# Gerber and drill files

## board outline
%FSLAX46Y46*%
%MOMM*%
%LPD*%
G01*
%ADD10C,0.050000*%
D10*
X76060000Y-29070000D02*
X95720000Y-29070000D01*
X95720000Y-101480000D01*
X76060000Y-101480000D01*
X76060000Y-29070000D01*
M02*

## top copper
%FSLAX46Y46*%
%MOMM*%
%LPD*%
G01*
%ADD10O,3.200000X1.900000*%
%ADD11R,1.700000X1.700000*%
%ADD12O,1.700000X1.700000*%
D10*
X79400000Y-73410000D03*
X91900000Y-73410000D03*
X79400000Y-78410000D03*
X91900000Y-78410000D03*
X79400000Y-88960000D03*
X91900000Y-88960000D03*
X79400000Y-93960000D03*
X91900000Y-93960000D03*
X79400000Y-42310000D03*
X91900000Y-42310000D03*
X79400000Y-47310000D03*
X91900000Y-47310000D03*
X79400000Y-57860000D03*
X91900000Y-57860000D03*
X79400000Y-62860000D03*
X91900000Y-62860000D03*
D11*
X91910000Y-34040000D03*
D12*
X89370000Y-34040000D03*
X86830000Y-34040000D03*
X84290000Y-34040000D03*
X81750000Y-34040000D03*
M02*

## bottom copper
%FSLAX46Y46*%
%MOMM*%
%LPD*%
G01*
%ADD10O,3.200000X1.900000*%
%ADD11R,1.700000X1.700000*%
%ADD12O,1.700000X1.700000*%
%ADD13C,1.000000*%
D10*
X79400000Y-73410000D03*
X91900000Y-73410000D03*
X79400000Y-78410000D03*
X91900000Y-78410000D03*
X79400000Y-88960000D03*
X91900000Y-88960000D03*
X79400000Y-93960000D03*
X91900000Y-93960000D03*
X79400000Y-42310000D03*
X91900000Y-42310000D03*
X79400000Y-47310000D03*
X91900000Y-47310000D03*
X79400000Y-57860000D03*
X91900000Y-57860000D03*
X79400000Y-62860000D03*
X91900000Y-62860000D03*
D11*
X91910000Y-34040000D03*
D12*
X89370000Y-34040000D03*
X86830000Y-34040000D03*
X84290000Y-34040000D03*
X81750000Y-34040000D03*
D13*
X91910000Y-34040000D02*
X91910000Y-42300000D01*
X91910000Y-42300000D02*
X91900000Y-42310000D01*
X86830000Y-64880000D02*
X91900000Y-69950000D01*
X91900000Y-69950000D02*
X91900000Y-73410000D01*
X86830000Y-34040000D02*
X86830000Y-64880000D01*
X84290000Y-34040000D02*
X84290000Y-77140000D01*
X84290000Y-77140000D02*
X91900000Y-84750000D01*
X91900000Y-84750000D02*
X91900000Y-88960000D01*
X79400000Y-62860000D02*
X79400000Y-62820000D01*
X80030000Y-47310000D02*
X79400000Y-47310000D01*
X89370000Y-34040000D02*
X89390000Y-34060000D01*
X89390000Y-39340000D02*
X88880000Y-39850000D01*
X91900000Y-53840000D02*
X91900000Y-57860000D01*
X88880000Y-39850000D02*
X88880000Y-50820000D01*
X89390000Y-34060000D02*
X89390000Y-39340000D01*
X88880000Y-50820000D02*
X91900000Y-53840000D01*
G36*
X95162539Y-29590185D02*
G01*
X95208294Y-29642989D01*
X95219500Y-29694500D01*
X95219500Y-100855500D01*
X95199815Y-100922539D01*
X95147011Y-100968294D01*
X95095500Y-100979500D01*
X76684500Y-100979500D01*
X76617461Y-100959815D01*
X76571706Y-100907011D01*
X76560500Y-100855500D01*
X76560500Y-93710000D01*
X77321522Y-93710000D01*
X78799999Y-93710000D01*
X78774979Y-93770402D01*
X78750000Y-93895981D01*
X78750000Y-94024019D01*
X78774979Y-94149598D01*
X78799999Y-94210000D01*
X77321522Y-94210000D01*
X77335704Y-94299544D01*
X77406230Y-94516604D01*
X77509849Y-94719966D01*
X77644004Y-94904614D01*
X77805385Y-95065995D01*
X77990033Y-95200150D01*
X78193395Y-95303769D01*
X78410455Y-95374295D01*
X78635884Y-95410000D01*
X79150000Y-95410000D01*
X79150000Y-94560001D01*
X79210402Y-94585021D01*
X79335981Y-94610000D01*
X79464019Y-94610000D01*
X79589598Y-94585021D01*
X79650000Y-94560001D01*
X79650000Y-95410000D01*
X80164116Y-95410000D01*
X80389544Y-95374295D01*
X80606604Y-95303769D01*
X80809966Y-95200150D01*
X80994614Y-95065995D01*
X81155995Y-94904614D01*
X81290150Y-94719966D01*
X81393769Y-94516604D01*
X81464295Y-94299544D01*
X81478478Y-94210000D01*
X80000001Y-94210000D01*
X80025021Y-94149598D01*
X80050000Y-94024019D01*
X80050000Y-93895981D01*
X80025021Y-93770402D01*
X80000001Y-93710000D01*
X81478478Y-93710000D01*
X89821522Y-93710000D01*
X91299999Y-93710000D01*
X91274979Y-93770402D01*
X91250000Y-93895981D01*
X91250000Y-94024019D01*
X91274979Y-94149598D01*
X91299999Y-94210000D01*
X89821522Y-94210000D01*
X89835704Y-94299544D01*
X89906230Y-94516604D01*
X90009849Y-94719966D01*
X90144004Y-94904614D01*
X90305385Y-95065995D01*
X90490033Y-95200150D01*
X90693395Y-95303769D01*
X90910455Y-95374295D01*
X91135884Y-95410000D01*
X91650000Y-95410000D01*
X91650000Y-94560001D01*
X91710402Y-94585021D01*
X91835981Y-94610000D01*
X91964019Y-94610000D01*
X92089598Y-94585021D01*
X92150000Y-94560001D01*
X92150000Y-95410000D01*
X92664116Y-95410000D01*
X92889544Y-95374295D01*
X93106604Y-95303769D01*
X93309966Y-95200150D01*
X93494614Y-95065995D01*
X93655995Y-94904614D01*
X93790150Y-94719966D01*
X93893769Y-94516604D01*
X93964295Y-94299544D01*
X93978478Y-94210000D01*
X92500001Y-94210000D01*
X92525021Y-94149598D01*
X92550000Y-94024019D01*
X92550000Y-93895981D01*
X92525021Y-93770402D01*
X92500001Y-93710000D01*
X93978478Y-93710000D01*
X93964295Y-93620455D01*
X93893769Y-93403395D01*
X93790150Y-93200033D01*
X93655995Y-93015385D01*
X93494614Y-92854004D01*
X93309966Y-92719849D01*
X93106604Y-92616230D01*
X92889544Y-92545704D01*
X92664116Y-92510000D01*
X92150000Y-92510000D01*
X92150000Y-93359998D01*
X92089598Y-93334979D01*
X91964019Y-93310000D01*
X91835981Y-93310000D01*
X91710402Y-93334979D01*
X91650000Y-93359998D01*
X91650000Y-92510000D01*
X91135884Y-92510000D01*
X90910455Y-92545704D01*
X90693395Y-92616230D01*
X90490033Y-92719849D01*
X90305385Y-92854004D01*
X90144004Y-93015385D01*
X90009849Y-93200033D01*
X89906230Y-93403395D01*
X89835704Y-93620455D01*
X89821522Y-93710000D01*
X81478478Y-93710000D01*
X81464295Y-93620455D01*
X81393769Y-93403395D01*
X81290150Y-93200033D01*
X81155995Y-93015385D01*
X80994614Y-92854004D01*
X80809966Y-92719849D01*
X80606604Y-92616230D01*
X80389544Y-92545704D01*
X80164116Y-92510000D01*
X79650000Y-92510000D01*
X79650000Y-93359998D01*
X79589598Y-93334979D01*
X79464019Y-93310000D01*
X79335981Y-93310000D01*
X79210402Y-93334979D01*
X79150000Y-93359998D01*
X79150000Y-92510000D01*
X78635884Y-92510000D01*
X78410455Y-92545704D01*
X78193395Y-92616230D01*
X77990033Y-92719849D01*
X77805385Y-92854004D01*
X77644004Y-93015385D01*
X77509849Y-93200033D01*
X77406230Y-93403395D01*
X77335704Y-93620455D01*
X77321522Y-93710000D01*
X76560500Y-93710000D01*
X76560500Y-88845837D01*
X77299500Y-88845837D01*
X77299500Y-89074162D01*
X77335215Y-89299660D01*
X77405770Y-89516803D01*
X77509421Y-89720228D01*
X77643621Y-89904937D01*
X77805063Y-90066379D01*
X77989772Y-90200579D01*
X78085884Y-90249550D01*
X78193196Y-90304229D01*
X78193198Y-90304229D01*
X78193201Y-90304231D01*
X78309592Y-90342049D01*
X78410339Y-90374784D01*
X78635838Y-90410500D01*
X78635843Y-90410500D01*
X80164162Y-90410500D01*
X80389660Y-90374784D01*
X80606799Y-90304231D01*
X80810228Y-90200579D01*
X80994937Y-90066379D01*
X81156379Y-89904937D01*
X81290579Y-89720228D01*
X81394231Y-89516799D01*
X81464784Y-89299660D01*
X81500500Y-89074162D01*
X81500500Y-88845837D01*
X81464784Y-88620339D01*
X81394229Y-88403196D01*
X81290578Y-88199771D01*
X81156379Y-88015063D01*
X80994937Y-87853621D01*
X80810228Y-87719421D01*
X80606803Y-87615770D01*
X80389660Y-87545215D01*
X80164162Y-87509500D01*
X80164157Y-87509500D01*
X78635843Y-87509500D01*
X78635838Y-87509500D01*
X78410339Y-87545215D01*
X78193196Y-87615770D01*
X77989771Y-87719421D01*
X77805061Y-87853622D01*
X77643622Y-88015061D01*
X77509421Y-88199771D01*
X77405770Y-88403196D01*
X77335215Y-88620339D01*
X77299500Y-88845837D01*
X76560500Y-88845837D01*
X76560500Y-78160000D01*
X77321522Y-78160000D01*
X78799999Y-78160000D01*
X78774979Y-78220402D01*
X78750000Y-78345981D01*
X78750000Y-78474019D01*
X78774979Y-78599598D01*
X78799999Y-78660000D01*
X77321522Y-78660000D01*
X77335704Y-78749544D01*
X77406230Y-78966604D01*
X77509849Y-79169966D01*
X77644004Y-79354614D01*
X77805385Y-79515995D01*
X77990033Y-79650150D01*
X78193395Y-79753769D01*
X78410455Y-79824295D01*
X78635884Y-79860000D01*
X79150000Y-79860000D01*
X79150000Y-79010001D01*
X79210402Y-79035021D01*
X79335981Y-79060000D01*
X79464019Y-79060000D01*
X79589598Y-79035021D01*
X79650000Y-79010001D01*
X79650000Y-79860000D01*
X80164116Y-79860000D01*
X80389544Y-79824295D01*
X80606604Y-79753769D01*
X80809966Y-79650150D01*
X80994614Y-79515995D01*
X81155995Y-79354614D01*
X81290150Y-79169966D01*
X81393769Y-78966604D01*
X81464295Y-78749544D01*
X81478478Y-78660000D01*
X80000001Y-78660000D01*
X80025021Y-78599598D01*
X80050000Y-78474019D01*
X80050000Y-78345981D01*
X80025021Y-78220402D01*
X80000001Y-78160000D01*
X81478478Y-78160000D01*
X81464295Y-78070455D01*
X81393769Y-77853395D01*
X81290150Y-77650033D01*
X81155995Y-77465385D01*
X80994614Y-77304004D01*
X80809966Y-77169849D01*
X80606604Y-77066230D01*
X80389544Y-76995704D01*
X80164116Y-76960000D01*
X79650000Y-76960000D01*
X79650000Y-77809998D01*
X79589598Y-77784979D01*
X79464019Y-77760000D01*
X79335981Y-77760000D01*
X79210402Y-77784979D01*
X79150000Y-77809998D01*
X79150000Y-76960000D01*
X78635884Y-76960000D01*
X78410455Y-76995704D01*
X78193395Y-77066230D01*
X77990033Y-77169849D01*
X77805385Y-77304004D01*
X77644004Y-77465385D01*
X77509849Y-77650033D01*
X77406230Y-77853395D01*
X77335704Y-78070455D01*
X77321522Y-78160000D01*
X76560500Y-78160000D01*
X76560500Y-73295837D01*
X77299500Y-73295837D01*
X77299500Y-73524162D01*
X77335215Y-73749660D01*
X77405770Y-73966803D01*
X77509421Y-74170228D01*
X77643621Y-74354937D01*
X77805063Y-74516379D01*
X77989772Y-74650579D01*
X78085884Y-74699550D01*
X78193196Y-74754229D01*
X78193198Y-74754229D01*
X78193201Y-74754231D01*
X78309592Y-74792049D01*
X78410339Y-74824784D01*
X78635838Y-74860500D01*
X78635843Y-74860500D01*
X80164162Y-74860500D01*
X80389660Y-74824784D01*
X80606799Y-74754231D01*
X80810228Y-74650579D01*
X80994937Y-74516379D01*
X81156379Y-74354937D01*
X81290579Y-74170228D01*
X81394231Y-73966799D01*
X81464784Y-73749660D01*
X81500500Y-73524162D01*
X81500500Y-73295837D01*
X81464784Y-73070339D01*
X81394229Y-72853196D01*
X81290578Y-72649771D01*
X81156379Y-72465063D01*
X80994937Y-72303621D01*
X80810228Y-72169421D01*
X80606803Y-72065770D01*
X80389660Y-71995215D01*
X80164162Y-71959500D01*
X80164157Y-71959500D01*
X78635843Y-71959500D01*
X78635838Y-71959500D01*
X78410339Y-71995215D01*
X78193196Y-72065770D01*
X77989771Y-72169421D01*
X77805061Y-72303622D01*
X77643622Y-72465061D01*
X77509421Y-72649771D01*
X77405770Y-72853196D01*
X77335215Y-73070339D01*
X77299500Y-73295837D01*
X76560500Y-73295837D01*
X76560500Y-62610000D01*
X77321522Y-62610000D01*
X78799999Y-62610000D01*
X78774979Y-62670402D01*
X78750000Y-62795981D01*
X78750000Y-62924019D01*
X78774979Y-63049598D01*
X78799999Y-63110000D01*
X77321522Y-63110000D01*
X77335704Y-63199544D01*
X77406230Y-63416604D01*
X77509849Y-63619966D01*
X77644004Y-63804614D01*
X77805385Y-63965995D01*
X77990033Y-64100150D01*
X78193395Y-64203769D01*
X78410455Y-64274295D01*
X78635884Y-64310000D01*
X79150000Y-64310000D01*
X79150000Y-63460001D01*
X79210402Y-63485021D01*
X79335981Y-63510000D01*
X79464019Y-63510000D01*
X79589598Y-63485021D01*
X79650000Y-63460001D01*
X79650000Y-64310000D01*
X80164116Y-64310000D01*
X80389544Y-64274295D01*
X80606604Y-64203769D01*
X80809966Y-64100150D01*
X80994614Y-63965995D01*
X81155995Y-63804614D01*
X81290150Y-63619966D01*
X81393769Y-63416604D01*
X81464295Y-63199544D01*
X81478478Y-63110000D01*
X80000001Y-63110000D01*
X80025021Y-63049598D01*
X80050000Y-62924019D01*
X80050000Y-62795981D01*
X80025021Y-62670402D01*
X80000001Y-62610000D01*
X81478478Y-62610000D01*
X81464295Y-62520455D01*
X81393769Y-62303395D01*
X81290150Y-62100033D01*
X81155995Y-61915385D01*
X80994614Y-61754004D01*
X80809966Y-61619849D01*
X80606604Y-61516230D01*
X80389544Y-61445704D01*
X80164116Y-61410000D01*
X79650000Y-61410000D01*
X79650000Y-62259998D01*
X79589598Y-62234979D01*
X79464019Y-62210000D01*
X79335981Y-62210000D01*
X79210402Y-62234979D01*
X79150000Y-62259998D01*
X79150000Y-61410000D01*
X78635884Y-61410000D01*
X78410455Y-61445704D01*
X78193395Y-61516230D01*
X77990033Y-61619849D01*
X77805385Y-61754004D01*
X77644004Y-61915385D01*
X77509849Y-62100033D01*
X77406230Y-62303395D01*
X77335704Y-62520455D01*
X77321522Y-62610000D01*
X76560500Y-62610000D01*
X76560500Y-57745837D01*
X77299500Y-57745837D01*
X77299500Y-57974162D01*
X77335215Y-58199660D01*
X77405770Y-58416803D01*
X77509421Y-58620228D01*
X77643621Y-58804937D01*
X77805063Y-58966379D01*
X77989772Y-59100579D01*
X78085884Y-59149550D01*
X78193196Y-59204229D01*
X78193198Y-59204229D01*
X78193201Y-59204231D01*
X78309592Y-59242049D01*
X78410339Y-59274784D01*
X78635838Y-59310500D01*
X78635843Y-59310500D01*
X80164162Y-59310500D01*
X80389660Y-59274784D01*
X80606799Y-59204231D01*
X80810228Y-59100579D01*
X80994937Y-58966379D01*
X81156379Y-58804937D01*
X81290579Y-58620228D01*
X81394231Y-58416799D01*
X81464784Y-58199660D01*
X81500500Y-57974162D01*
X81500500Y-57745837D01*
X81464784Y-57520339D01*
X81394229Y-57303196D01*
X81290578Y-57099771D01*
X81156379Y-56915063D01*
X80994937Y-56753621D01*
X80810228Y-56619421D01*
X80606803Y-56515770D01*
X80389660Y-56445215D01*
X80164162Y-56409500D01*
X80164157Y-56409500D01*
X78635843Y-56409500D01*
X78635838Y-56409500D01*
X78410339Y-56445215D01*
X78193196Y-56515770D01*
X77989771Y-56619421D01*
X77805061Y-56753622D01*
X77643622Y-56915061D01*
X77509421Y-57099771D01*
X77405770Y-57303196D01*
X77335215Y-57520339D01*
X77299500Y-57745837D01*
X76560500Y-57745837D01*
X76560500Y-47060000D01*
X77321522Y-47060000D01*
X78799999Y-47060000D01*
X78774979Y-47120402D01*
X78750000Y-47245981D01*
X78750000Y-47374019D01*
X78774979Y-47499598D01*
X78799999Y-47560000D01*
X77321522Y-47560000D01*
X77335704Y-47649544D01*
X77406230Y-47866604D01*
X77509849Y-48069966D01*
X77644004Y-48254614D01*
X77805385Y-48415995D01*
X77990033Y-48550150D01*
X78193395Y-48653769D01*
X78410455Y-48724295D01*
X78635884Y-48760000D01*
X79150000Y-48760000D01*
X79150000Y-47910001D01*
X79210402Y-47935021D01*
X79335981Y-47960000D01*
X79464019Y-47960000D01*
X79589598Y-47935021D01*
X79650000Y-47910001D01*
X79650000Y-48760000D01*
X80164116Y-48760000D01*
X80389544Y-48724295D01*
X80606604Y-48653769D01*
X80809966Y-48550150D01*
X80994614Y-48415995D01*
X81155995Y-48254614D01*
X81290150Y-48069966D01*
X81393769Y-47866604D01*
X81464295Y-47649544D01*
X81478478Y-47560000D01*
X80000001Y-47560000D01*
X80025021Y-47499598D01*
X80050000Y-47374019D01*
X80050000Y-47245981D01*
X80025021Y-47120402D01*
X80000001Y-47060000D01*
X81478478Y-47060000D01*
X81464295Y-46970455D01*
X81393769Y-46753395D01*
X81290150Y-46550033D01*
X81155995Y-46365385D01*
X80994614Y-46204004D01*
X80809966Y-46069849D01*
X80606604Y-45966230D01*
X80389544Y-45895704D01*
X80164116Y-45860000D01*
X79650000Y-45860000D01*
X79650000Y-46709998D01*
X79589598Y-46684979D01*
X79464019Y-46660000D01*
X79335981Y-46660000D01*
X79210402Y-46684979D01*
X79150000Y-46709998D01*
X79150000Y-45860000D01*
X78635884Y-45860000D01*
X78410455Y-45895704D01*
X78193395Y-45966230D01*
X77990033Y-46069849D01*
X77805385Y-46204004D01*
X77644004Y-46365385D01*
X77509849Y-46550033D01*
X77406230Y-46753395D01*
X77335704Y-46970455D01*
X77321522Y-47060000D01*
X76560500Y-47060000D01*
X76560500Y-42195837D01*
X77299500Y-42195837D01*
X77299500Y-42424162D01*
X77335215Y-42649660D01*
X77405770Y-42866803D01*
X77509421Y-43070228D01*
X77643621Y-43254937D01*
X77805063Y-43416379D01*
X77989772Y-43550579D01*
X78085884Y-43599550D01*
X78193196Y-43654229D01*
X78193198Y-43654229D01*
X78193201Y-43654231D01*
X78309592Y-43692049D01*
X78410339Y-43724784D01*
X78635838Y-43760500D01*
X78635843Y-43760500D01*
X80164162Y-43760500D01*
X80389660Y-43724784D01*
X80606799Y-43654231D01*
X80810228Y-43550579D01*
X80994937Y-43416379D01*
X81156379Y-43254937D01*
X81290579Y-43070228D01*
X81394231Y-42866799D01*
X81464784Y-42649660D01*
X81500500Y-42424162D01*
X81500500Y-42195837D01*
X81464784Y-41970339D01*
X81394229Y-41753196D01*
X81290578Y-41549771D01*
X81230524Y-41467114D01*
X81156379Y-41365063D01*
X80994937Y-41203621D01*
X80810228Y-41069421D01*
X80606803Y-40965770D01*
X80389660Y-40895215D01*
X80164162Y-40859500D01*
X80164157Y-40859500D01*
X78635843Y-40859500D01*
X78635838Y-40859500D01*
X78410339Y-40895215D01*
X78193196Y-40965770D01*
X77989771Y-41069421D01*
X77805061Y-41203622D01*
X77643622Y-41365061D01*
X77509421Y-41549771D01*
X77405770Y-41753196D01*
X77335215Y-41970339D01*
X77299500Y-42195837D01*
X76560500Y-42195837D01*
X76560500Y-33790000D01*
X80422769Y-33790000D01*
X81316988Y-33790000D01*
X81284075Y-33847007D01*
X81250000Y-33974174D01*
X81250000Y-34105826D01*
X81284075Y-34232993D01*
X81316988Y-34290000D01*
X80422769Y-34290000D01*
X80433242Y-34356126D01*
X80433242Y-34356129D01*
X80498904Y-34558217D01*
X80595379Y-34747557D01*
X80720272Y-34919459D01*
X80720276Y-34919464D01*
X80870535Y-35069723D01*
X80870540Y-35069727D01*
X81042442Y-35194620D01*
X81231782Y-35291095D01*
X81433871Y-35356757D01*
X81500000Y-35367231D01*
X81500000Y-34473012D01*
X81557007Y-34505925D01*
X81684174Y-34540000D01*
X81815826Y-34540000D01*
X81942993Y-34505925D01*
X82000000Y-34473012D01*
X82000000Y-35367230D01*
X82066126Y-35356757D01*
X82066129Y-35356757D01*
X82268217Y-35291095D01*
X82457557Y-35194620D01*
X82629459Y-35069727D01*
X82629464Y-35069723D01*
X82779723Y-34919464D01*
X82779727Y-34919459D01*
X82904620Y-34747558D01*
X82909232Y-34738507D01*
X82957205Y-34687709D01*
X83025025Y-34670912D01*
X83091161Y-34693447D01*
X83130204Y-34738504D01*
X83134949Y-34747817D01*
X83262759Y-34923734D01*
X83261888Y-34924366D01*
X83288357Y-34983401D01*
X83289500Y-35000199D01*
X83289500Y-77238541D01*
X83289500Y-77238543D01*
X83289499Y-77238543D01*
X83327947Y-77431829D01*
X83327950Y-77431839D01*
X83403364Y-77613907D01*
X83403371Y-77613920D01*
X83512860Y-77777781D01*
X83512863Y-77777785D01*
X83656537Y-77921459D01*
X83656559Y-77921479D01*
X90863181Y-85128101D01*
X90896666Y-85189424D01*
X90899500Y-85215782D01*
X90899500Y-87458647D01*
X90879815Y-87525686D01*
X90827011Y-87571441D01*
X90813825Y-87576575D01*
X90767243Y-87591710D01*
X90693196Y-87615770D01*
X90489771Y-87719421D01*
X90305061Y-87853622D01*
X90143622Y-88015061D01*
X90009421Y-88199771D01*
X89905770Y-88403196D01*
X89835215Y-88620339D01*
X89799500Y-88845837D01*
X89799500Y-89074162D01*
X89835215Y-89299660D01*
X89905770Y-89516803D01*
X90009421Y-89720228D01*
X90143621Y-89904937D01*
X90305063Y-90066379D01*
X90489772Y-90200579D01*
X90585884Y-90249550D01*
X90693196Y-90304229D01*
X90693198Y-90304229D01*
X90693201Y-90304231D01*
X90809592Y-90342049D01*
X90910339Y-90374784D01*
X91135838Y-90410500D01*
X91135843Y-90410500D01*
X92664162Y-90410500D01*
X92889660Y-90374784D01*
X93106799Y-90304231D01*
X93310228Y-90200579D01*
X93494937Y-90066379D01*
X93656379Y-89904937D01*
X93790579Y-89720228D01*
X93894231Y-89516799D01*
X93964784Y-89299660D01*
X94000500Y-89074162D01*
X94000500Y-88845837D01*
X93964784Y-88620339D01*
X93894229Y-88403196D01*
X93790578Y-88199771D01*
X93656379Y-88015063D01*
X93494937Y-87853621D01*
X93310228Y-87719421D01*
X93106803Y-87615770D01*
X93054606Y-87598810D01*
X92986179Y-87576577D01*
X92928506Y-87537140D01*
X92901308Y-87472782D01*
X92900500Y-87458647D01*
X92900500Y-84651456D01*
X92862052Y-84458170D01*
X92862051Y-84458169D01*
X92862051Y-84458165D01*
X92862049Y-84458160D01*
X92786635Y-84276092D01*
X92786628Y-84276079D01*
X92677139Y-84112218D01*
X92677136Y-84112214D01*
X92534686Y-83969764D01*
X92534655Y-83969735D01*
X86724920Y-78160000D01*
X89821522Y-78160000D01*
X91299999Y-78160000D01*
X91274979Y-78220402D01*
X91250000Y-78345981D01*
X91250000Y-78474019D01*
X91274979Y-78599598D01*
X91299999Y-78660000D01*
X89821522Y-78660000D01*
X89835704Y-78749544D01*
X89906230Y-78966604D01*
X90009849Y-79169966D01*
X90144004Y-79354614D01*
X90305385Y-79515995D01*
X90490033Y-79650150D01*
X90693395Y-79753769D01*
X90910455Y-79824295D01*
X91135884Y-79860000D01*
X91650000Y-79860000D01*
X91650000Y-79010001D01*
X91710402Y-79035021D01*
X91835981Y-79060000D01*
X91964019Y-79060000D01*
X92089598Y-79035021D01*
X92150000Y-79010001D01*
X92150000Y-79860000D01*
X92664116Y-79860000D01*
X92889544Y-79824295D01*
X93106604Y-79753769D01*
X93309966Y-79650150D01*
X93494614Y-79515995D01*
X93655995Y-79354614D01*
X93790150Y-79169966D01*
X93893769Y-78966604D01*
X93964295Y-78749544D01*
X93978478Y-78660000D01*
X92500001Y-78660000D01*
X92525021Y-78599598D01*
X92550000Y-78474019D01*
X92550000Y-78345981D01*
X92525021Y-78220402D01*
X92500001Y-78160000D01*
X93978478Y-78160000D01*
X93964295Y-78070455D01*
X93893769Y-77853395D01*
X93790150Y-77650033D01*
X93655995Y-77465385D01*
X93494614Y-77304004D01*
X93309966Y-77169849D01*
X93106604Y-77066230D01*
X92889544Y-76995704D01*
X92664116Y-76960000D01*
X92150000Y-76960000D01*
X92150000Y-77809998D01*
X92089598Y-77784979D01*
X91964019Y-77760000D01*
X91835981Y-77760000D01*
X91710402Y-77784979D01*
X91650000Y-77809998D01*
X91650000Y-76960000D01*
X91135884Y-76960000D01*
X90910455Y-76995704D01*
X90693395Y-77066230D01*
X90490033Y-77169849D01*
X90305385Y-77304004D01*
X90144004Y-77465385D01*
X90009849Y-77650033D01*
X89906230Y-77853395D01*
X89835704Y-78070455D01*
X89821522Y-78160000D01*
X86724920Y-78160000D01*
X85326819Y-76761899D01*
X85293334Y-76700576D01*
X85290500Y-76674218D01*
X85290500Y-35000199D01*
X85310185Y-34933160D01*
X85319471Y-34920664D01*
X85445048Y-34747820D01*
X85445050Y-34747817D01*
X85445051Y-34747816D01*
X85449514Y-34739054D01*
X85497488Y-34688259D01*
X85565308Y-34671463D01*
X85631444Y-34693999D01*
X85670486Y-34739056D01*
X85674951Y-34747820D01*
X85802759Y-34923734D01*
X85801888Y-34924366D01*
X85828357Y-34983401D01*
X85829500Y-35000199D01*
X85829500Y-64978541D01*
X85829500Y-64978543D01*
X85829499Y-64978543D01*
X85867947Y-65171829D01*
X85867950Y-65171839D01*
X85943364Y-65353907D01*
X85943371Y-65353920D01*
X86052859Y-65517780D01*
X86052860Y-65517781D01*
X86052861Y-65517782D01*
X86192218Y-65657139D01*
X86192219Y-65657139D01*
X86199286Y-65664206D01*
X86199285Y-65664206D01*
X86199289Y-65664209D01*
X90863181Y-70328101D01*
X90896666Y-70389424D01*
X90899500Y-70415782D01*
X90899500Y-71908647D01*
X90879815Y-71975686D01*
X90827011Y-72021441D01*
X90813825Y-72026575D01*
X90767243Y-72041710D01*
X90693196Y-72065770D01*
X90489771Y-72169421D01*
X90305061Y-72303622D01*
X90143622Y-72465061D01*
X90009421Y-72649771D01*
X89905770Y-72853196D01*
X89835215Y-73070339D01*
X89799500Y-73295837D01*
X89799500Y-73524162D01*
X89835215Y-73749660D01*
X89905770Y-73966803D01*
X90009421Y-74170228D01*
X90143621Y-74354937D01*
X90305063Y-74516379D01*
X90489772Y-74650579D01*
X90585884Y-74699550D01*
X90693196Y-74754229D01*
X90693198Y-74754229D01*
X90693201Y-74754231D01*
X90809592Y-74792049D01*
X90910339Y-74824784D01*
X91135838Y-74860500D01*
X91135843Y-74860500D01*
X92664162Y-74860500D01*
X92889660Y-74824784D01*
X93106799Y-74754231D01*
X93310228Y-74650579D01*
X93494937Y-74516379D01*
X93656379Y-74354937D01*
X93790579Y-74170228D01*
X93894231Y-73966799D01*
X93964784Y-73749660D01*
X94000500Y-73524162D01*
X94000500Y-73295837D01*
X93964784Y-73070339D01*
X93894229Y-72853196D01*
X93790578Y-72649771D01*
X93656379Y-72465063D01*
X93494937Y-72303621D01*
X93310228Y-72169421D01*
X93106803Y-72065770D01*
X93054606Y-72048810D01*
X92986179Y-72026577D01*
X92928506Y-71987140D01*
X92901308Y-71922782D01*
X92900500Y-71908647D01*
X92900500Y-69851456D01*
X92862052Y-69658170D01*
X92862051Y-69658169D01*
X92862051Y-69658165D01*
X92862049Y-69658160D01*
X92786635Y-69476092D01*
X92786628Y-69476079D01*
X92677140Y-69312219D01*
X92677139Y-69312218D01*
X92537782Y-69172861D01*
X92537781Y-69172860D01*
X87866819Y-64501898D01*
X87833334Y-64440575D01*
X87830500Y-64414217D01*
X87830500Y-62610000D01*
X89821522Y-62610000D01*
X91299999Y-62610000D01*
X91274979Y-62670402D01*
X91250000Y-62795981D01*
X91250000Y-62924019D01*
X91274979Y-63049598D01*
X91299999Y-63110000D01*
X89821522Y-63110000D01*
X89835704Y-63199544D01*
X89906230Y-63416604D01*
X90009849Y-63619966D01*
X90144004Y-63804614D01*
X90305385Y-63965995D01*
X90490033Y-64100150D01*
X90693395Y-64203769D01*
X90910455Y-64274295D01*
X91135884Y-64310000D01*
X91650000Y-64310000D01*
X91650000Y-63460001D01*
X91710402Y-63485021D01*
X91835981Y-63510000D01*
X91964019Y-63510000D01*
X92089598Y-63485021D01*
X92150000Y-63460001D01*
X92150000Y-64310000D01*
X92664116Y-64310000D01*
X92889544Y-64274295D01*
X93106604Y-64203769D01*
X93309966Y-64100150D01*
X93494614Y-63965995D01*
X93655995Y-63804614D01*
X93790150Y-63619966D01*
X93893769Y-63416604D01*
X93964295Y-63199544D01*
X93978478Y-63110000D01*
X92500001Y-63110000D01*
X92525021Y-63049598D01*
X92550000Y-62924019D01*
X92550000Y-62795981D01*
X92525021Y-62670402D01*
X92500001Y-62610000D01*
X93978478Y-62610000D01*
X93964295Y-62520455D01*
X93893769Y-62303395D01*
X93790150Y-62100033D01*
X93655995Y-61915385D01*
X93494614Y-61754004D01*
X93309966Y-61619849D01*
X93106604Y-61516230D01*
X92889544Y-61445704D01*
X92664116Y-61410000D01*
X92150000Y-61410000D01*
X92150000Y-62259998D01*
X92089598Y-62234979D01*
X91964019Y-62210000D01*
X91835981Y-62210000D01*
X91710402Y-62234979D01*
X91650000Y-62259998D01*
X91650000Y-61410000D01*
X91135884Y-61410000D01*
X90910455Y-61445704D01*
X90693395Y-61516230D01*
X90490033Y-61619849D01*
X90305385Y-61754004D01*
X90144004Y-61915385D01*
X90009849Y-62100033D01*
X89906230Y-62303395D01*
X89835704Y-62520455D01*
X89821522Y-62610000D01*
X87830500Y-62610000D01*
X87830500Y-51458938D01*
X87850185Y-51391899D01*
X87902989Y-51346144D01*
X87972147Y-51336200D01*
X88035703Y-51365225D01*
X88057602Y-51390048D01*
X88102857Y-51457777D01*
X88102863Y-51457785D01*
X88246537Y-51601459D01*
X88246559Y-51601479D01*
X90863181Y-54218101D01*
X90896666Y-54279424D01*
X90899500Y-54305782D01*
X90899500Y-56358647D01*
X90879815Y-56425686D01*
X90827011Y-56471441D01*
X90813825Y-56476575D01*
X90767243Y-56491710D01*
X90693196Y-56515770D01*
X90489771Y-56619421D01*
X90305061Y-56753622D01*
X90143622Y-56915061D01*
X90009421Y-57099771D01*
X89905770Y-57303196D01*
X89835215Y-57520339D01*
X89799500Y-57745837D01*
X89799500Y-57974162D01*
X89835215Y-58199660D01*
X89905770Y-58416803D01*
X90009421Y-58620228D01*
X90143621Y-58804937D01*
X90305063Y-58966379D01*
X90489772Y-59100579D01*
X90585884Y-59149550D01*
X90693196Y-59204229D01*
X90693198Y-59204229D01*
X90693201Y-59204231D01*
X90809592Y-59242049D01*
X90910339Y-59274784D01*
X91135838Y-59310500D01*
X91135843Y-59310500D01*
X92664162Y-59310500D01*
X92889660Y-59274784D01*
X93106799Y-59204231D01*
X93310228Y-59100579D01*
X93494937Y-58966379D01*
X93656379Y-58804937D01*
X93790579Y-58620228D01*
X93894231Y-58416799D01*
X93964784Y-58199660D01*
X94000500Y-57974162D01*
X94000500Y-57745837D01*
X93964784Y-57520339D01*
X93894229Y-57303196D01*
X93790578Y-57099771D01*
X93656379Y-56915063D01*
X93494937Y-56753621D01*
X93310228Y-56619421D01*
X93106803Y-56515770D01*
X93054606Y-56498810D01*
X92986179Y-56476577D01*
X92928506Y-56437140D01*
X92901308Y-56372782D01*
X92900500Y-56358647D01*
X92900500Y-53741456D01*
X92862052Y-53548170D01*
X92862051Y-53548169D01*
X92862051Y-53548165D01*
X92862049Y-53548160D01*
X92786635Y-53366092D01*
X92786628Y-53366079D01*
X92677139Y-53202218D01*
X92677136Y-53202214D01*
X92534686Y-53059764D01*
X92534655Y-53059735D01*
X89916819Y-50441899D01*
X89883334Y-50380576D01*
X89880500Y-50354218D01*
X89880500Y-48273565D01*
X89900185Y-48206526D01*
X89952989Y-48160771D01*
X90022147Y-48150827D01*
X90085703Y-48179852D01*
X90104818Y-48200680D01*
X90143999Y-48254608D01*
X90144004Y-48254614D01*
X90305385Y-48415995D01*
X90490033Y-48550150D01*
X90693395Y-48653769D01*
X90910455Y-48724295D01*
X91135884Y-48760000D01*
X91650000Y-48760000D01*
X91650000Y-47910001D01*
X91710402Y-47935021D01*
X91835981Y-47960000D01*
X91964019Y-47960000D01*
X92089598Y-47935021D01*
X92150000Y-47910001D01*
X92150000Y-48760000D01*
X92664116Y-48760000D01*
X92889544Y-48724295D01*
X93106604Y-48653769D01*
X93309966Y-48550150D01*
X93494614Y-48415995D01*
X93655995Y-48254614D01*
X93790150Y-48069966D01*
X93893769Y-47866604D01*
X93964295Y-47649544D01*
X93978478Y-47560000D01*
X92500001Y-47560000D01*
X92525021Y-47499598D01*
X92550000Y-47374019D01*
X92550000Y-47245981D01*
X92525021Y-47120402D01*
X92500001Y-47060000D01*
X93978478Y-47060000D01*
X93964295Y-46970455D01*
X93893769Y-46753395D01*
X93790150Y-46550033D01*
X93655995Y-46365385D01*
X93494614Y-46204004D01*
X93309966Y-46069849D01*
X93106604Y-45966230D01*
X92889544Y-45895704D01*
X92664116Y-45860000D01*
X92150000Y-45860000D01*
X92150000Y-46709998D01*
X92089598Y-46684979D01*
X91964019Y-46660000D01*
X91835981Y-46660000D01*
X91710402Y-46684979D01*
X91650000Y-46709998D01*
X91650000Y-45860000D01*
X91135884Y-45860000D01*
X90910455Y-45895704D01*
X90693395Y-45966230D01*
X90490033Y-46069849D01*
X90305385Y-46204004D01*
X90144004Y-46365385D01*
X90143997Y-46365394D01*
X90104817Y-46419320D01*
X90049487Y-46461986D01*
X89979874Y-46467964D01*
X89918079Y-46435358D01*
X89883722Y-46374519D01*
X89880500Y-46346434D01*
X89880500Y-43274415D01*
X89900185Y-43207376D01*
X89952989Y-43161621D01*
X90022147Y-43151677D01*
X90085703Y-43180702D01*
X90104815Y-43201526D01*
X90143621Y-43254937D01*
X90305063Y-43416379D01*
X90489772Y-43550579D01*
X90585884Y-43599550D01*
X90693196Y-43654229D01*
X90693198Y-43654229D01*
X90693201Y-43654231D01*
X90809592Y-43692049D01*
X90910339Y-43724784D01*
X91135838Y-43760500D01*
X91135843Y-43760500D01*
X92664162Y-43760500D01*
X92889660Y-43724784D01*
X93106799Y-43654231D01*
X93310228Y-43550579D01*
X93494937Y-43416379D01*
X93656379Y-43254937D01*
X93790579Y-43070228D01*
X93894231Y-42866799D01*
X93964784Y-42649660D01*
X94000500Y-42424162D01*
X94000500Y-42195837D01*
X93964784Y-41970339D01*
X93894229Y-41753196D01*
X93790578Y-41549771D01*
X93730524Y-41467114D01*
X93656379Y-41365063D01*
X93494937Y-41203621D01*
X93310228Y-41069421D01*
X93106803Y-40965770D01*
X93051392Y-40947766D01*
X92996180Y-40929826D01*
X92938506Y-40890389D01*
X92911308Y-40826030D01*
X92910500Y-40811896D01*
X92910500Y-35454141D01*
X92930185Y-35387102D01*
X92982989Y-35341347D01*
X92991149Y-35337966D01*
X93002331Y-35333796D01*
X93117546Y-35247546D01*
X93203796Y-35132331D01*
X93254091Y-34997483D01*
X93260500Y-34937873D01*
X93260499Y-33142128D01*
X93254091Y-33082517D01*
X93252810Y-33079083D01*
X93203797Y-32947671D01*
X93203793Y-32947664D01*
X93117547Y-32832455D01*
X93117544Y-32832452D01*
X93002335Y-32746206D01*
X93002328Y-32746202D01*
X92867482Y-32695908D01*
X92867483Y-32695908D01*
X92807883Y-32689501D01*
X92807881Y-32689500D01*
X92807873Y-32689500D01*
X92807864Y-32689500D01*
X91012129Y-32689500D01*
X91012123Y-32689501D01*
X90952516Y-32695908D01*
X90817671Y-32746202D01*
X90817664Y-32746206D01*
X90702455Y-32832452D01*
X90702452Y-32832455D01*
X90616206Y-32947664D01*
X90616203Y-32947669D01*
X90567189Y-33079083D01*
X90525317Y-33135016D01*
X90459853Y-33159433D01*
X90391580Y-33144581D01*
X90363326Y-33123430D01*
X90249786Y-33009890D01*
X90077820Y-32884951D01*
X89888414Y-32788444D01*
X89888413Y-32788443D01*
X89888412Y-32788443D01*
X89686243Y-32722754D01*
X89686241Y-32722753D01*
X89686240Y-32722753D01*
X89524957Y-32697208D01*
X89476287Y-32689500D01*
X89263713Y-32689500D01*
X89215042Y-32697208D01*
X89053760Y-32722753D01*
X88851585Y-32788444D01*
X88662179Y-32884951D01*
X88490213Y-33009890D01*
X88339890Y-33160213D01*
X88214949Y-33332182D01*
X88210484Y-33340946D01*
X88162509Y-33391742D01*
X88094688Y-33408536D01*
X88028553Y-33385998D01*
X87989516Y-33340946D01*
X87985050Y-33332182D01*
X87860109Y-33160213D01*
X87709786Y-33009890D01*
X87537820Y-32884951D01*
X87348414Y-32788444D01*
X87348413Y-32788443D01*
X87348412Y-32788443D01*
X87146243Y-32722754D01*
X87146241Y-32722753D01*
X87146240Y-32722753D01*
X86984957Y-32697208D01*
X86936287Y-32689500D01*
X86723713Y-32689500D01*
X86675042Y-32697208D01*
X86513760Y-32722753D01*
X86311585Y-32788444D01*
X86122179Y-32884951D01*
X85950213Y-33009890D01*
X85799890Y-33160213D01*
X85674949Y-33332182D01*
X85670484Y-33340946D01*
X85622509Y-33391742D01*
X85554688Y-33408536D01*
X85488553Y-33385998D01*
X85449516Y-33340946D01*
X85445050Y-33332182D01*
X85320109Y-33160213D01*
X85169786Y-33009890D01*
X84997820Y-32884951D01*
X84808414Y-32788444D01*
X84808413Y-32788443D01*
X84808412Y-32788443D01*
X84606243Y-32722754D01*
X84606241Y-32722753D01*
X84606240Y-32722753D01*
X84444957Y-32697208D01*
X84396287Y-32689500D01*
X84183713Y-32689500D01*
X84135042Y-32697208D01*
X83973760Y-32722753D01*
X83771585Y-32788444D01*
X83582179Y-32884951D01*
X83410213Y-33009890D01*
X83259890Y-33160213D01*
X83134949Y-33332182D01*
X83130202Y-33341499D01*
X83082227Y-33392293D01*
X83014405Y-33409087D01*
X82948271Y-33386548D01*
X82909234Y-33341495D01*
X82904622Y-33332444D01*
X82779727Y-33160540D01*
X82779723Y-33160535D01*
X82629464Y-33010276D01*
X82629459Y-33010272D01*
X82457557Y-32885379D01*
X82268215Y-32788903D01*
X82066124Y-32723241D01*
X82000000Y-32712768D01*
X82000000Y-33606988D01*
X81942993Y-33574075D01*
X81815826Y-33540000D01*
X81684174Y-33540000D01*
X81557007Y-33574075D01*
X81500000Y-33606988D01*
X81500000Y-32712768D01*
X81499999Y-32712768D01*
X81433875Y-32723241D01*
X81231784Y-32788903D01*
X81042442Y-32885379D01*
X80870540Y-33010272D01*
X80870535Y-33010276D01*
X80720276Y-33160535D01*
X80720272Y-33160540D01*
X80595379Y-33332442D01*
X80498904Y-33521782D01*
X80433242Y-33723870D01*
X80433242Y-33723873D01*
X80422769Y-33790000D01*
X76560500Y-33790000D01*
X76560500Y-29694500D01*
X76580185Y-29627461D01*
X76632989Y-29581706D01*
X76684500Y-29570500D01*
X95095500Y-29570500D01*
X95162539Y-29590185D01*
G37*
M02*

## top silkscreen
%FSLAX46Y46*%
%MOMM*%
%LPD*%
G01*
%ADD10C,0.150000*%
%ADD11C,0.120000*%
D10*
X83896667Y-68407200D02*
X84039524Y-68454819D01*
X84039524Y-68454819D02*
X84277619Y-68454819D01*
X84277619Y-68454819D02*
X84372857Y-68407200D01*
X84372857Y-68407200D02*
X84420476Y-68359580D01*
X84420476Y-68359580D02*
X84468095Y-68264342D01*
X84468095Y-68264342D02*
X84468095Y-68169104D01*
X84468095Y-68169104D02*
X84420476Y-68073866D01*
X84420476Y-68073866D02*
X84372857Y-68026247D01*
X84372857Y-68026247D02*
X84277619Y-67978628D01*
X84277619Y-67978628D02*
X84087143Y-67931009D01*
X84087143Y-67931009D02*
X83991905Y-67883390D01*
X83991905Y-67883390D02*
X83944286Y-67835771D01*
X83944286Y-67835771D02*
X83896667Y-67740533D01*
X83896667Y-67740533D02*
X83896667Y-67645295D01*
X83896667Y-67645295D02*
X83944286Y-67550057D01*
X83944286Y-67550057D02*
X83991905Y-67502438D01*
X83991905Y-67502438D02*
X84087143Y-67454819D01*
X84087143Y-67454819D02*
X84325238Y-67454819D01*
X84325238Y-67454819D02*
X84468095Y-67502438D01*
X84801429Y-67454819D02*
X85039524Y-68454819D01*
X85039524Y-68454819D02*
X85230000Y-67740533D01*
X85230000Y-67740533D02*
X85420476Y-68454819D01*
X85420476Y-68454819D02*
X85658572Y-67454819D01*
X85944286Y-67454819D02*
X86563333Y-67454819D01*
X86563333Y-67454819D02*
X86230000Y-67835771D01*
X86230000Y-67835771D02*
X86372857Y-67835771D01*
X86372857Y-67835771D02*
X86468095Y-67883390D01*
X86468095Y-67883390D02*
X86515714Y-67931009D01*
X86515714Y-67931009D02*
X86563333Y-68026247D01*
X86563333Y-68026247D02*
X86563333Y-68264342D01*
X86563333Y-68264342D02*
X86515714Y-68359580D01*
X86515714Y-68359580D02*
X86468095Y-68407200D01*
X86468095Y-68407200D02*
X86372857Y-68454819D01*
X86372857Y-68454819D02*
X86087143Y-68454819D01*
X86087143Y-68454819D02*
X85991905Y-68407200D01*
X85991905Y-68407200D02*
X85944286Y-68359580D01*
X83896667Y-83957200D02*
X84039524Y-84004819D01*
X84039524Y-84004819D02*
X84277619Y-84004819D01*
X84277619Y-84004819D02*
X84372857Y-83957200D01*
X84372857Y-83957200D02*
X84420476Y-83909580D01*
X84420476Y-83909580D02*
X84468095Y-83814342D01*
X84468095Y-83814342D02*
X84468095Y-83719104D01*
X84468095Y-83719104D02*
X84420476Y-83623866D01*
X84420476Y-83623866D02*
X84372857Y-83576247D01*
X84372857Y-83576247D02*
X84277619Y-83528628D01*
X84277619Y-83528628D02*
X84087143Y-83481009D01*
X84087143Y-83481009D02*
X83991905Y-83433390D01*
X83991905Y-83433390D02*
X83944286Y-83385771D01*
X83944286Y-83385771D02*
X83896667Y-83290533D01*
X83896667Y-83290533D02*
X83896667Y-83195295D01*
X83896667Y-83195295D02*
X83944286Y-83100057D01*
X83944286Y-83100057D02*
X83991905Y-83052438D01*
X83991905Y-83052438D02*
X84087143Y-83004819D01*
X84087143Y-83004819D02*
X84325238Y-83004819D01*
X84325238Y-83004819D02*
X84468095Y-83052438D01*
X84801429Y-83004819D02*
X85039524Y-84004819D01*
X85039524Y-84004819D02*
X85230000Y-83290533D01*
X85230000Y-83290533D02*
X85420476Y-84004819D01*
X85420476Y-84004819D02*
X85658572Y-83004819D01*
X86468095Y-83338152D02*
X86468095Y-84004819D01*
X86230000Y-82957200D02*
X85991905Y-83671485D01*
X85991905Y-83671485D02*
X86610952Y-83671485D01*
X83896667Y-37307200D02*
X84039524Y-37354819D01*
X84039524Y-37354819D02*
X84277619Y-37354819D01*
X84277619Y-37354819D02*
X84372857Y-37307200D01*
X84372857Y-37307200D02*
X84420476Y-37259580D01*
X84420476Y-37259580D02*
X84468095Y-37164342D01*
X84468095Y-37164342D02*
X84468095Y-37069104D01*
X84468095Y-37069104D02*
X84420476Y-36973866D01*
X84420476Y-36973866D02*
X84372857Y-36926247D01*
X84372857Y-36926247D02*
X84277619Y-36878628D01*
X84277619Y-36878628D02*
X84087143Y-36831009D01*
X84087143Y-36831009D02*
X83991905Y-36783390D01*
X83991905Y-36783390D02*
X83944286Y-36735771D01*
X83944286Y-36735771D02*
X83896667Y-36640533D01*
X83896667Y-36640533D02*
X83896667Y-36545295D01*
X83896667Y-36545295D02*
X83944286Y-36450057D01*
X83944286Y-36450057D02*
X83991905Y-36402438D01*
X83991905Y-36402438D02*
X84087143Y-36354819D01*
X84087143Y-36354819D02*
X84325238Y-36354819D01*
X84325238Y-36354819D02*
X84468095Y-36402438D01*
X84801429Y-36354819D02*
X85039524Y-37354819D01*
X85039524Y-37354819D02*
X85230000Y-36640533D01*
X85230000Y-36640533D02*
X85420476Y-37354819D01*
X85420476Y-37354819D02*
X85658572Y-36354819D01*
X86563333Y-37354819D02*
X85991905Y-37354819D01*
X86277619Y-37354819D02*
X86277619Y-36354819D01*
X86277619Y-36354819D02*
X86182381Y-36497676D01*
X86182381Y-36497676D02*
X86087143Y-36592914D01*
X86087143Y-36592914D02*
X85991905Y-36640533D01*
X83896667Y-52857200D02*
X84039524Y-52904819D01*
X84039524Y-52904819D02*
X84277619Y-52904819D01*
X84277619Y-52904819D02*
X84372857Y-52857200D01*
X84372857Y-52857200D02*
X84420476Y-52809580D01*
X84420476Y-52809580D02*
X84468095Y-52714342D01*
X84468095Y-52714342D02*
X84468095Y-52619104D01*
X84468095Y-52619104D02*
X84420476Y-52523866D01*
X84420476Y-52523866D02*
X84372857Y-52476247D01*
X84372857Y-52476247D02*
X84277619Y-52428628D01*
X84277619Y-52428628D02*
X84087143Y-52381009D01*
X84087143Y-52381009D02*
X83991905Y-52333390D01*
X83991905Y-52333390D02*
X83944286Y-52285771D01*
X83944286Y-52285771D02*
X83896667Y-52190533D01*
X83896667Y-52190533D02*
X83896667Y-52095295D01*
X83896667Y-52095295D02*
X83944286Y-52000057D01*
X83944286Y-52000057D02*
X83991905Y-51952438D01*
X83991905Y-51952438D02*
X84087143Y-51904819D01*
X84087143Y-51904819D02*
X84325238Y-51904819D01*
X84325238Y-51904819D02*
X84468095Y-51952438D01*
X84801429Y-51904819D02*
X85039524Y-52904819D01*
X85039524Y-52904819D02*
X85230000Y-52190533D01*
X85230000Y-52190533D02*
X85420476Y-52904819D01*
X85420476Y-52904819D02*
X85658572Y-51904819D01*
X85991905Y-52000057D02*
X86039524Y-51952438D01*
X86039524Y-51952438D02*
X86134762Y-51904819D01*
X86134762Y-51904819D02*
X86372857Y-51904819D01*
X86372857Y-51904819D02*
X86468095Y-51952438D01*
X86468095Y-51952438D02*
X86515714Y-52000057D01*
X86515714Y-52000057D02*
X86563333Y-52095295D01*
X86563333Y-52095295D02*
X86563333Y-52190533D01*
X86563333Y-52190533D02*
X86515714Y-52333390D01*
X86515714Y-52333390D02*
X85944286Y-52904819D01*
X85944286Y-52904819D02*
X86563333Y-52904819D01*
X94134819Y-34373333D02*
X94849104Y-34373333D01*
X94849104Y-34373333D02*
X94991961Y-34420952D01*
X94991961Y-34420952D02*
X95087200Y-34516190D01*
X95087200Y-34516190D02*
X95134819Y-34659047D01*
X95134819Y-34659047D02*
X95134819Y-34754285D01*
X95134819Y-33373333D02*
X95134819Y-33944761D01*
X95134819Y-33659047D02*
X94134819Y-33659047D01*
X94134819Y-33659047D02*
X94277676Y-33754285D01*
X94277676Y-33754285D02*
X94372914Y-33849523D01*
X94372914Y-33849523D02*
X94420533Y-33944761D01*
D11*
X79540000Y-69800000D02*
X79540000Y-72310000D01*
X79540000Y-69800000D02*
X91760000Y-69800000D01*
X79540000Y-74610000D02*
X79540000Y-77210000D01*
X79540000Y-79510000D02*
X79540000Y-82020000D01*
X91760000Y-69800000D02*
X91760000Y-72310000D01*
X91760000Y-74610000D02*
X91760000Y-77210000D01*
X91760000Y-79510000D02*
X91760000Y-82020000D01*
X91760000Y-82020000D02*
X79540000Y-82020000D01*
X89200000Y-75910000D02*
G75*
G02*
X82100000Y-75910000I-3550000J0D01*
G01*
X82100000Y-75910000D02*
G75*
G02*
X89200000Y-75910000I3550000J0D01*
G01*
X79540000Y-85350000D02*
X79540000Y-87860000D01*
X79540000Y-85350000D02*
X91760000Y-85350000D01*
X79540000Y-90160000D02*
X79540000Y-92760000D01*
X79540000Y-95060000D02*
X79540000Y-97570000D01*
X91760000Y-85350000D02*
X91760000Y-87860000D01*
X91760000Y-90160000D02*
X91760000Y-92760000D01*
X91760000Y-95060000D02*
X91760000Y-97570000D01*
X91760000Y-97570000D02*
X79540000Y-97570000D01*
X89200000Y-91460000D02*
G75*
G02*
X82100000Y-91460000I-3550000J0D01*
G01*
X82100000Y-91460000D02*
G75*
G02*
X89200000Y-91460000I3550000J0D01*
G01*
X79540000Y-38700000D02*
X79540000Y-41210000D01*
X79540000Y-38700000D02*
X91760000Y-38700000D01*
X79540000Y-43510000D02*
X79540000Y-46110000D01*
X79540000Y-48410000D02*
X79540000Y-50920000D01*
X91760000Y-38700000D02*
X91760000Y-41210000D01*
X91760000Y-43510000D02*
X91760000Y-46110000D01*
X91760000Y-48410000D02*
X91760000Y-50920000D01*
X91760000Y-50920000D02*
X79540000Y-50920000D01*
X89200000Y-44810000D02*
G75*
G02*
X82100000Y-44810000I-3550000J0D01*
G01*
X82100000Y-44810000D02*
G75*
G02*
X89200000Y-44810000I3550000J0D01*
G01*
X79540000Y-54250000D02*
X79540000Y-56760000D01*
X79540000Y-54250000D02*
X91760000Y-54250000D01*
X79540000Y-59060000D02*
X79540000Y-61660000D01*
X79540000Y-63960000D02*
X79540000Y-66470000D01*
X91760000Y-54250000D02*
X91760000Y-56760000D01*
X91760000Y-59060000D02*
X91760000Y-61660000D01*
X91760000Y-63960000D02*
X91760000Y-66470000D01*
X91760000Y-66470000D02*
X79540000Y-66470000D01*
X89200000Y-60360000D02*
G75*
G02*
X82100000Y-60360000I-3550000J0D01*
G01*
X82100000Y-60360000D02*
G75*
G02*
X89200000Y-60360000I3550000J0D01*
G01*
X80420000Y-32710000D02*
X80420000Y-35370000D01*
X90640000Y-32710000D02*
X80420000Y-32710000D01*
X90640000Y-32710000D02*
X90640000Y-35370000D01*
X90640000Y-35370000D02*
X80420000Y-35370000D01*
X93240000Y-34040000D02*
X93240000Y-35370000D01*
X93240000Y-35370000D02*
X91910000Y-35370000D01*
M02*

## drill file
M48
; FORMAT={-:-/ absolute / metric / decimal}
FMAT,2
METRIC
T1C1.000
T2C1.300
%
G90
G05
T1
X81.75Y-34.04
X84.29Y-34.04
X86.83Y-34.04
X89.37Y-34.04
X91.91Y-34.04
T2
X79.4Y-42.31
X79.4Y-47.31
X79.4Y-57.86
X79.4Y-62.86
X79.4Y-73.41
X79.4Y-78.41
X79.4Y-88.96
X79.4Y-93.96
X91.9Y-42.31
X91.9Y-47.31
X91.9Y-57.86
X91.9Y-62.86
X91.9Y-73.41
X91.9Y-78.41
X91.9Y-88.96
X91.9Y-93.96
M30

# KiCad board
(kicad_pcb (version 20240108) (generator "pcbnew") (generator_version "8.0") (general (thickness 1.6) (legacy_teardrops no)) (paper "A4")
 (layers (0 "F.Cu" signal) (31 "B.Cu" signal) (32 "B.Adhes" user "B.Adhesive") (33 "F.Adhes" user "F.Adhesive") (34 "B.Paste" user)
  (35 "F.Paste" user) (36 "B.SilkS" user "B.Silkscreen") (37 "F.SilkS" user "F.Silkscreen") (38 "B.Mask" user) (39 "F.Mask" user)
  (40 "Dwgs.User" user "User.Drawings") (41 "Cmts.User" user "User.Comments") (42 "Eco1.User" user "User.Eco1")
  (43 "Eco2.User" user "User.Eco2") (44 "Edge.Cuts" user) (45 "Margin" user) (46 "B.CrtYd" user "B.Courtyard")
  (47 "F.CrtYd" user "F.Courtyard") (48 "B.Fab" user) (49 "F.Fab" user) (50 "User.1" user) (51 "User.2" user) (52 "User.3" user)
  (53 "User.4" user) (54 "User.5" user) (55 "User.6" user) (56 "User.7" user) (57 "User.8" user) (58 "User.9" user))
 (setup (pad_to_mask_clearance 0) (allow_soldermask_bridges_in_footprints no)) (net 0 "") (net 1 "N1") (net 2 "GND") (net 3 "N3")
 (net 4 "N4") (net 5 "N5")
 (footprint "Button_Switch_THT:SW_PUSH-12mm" (layer "F.Cu") (at 79.4 73.41)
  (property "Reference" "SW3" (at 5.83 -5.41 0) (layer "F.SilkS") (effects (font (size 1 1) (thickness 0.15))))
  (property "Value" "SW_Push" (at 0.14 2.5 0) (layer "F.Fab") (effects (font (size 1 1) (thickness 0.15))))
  (fp_line (start 0.14 -3.61) (end 0.14 -1.1) (stroke (width 0.12) (type default)) (layer "F.SilkS"))
  (fp_line (start 0.14 -3.61) (end 12.36 -3.61) (stroke (width 0.12) (type default)) (layer "F.SilkS"))
  (fp_line (start 0.14 1.2) (end 0.14 3.8) (stroke (width 0.12) (type default)) (layer "F.SilkS"))
  (fp_line (start 0.14 6.1) (end 0.14 8.61) (stroke (width 0.12) (type default)) (layer "F.SilkS"))
  (fp_line (start 12.36 -3.61) (end 12.36 -1.1) (stroke (width 0.12) (type default)) (layer "F.SilkS"))
  (fp_line (start 12.36 1.2) (end 12.36 3.8) (stroke (width 0.12) (type default)) (layer "F.SilkS"))
  (fp_line (start 12.36 6.1) (end 12.36 8.61) (stroke (width 0.12) (type default)) (layer "F.SilkS"))
  (fp_line (start 12.36 8.61) (end 0.14 8.61) (stroke (width 0.12) (type default)) (layer "F.SilkS"))
  (fp_circle (center 6.25 2.5) (end 9.8 2.5) (stroke (width 0.12) (type default)) (fill none) (layer "F.SilkS"))
  (pad "1" thru_hole oval (at 0 0) (size 3.2 1.9) (drill 1.3) (layers "*.Cu" "*.Mask") (remove_unused_layers no) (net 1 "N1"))
  (pad "1" thru_hole oval (at 12.5 0) (size 3.2 1.9) (drill 1.3) (layers "*.Cu" "*.Mask") (remove_unused_layers no) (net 1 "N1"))
  (pad "2" thru_hole oval (at 0 5) (size 3.2 1.9) (drill 1.3) (layers "*.Cu" "*.Mask") (remove_unused_layers no) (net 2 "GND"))
  (pad "2" thru_hole oval (at 12.5 5) (size 3.2 1.9) (drill 1.3) (layers "*.Cu" "*.Mask") (remove_unused_layers no) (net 2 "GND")))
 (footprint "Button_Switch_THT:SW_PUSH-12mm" (layer "F.Cu") (at 79.4 88.96)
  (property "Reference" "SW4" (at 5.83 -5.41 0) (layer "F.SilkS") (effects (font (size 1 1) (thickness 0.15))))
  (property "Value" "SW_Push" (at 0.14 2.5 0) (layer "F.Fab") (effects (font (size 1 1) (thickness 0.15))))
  (fp_line (start 0.14 -3.61) (end 0.14 -1.1) (stroke (width 0.12) (type default)) (layer "F.SilkS"))
  (fp_line (start 0.14 -3.61) (end 12.36 -3.61) (stroke (width 0.12) (type default)) (layer "F.SilkS"))
  (fp_line (start 0.14 1.2) (end 0.14 3.8) (stroke (width 0.12) (type default)) (layer "F.SilkS"))
  (fp_line (start 0.14 6.1) (end 0.14 8.61) (stroke (width 0.12) (type default)) (layer "F.SilkS"))
  (fp_line (start 12.36 -3.61) (end 12.36 -1.1) (stroke (width 0.12) (type default)) (layer "F.SilkS"))
  (fp_line (start 12.36 1.2) (end 12.36 3.8) (stroke (width 0.12) (type default)) (layer "F.SilkS"))
  (fp_line (start 12.36 6.1) (end 12.36 8.61) (stroke (width 0.12) (type default)) (layer "F.SilkS"))
  (fp_line (start 12.36 8.61) (end 0.14 8.61) (stroke (width 0.12) (type default)) (layer "F.SilkS"))
  (fp_circle (center 6.25 2.5) (end 9.8 2.5) (stroke (width 0.12) (type default)) (fill none) (layer "F.SilkS"))
  (pad "1" thru_hole oval (at 0 0) (size 3.2 1.9) (drill 1.3) (layers "*.Cu" "*.Mask") (remove_unused_layers no) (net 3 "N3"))
  (pad "1" thru_hole oval (at 12.5 0) (size 3.2 1.9) (drill 1.3) (layers "*.Cu" "*.Mask") (remove_unused_layers no) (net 3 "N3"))
  (pad "2" thru_hole oval (at 0 5) (size 3.2 1.9) (drill 1.3) (layers "*.Cu" "*.Mask") (remove_unused_layers no) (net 2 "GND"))
  (pad "2" thru_hole oval (at 12.5 5) (size 3.2 1.9) (drill 1.3) (layers "*.Cu" "*.Mask") (remove_unused_layers no) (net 2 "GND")))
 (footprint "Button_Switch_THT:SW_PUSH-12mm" (layer "F.Cu") (at 79.4 42.31)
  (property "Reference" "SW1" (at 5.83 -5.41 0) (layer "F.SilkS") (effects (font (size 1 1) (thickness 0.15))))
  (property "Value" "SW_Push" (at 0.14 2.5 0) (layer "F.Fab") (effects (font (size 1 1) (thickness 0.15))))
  (fp_line (start 0.14 -3.61) (end 0.14 -1.1) (stroke (width 0.12) (type default)) (layer "F.SilkS"))
  (fp_line (start 0.14 -3.61) (end 12.36 -3.61) (stroke (width 0.12) (type default)) (layer "F.SilkS"))
  (fp_line (start 0.14 1.2) (end 0.14 3.8) (stroke (width 0.12) (type default)) (layer "F.SilkS"))
  (fp_line (start 0.14 6.1) (end 0.14 8.61) (stroke (width 0.12) (type default)) (layer "F.SilkS"))
  (fp_line (start 12.36 -3.61) (end 12.36 -1.1) (stroke (width 0.12) (type default)) (layer "F.SilkS"))
  (fp_line (start 12.36 1.2) (end 12.36 3.8) (stroke (width 0.12) (type default)) (layer "F.SilkS"))
  (fp_line (start 12.36 6.1) (end 12.36 8.61) (stroke (width 0.12) (type default)) (layer "F.SilkS"))
  (fp_line (start 12.36 8.61) (end 0.14 8.61) (stroke (width 0.12) (type default)) (layer "F.SilkS"))
  (fp_circle (center 6.25 2.5) (end 9.8 2.5) (stroke (width 0.12) (type default)) (fill none) (layer "F.SilkS"))
  (pad "1" thru_hole oval (at 0 0) (size 3.2 1.9) (drill 1.3) (layers "*.Cu" "*.Mask") (remove_unused_layers no) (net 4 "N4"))
  (pad "1" thru_hole oval (at 12.5 0) (size 3.2 1.9) (drill 1.3) (layers "*.Cu" "*.Mask") (remove_unused_layers no) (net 4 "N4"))
  (pad "2" thru_hole oval (at 0 5) (size 3.2 1.9) (drill 1.3) (layers "*.Cu" "*.Mask") (remove_unused_layers no) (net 2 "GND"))
  (pad "2" thru_hole oval (at 12.5 5) (size 3.2 1.9) (drill 1.3) (layers "*.Cu" "*.Mask") (remove_unused_layers no) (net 2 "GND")))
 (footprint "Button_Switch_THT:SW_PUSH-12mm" (layer "F.Cu") (at 79.4 57.86)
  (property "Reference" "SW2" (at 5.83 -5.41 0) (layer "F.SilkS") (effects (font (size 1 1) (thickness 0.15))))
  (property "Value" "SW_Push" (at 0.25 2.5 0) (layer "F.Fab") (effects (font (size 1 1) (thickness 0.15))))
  (fp_line (start 0.14 -3.61) (end 0.14 -1.1) (stroke (width 0.12) (type default)) (layer "F.SilkS"))
  (fp_line (start 0.14 -3.61) (end 12.36 -3.61) (stroke (width 0.12) (type default)) (layer "F.SilkS"))
  (fp_line (start 0.14 1.2) (end 0.14 3.8) (stroke (width 0.12) (type default)) (layer "F.SilkS"))
  (fp_line (start 0.14 6.1) (end 0.14 8.61) (stroke (width 0.12) (type default)) (layer "F.SilkS"))
  (fp_line (start 12.36 -3.61) (end 12.36 -1.1) (stroke (width 0.12) (type default)) (layer "F.SilkS"))
  (fp_line (start 12.36 1.2) (end 12.36 3.8) (stroke (width 0.12) (type default)) (layer "F.SilkS"))
  (fp_line (start 12.36 6.1) (end 12.36 8.61) (stroke (width 0.12) (type default)) (layer "F.SilkS"))
  (fp_line (start 12.36 8.61) (end 0.14 8.61) (stroke (width 0.12) (type default)) (layer "F.SilkS"))
  (fp_circle (center 6.25 2.5) (end 9.8 2.5) (stroke (width 0.12) (type default)) (fill none) (layer "F.SilkS"))
  (pad "1" thru_hole oval (at 0 0) (size 3.2 1.9) (drill 1.3) (layers "*.Cu" "*.Mask") (remove_unused_layers no) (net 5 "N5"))
  (pad "1" thru_hole oval (at 12.5 0) (size 3.2 1.9) (drill 1.3) (layers "*.Cu" "*.Mask") (remove_unused_layers no) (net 5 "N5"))
  (pad "2" thru_hole oval (at 0 5) (size 3.2 1.9) (drill 1.3) (layers "*.Cu" "*.Mask") (remove_unused_layers no) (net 2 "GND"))
  (pad "2" thru_hole oval (at 12.5 5) (size 3.2 1.9) (drill 1.3) (layers "*.Cu" "*.Mask") (remove_unused_layers no) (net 2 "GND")))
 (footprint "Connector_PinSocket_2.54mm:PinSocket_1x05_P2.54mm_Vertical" (layer "F.Cu") (at 91.91 34.04 -90)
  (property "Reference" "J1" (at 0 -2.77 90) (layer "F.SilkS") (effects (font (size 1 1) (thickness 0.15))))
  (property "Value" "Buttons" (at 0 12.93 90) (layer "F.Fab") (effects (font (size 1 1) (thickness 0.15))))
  (fp_line (start -1.33 11.49) (end 1.33 11.49) (stroke (width 0.12) (type solid)) (layer "F.SilkS"))
  (fp_line (start -1.33 1.27) (end -1.33 11.49) (stroke (width 0.12) (type solid)) (layer "F.SilkS"))
  (fp_line (start -1.33 1.27) (end 1.33 1.27) (stroke (width 0.12) (type solid)) (layer "F.SilkS"))
  (fp_line (start 1.33 1.27) (end 1.33 11.49) (stroke (width 0.12) (type solid)) (layer "F.SilkS"))
  (fp_line (start 0 -1.33) (end 1.33 -1.33) (stroke (width 0.12) (type solid)) (layer "F.SilkS"))
  (fp_line (start 1.33 -1.33) (end 1.33 0) (stroke (width 0.12) (type solid)) (layer "F.SilkS"))
  (pad "1" thru_hole rect (at 0 0 270) (size 1.7 1.7) (drill 1) (layers "*.Cu" "*.Mask") (remove_unused_layers no) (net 4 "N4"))
  (pad "2" thru_hole oval (at 0 2.54 270) (size 1.7 1.7) (drill 1) (layers "*.Cu" "*.Mask") (remove_unused_layers no) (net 5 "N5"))
  (pad "3" thru_hole oval (at 0 5.08 270) (size 1.7 1.7) (drill 1) (layers "*.Cu" "*.Mask") (remove_unused_layers no) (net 1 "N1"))
  (pad "4" thru_hole oval (at 0 7.62 270) (size 1.7 1.7) (drill 1) (layers "*.Cu" "*.Mask") (remove_unused_layers no) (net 3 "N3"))
  (pad "5" thru_hole oval (at 0 10.16 270) (size 1.7 1.7) (drill 1) (layers "*.Cu" "*.Mask") (remove_unused_layers no) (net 2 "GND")))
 (gr_rect (start 76.06 29.07) (end 95.72 101.48) (stroke (width 0.05) (type default)) (fill none) (layer "Edge.Cuts"))
 (segment (start 91.91 34.04) (end 91.91 42.3) (width 1) (layer "B.Cu") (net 4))
 (segment (start 91.91 42.3) (end 91.9 42.31) (width 1) (layer "B.Cu") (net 4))
 (segment (start 86.83 64.88) (end 91.9 69.95) (width 1) (layer "B.Cu") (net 1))
 (segment (start 91.9 69.95) (end 91.9 73.41) (width 1) (layer "B.Cu") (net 1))
 (segment (start 86.83 34.04) (end 86.83 64.88) (width 1) (layer "B.Cu") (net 1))
 (segment (start 84.29 34.04) (end 84.29 77.14) (width 1) (layer "B.Cu") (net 3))
 (segment (start 84.29 77.14) (end 91.9 84.75) (width 1) (layer "B.Cu") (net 3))
 (segment (start 91.9 84.75) (end 91.9 88.96) (width 1) (layer "B.Cu") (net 3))
 (segment (start 79.4 62.86) (end 79.4 62.82) (width 1) (layer "B.Cu") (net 2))
 (segment (start 80.03 47.31) (end 79.4 47.31) (width 1) (layer "B.Cu") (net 2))
 (segment (start 89.37 34.04) (end 89.39 34.06) (width 1) (layer "B.Cu") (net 5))
 (segment (start 89.39 39.34) (end 88.88 39.85) (width 1) (layer "B.Cu") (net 5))
 (segment (start 91.9 53.84) (end 91.9 57.86) (width 1) (layer "B.Cu") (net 5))
 (segment (start 88.88 39.85) (end 88.88 50.82) (width 1) (layer "B.Cu") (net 5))
 (segment (start 89.39 34.06) (end 89.39 39.34) (width 1) (layer "B.Cu") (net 5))
 (segment (start 88.88 50.82) (end 91.9 53.84) (width 1) (layer "B.Cu") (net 5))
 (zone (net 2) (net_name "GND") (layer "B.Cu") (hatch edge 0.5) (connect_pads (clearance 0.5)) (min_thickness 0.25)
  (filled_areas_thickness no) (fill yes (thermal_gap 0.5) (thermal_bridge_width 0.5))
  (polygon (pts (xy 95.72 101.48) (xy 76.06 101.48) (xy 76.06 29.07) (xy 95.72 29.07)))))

